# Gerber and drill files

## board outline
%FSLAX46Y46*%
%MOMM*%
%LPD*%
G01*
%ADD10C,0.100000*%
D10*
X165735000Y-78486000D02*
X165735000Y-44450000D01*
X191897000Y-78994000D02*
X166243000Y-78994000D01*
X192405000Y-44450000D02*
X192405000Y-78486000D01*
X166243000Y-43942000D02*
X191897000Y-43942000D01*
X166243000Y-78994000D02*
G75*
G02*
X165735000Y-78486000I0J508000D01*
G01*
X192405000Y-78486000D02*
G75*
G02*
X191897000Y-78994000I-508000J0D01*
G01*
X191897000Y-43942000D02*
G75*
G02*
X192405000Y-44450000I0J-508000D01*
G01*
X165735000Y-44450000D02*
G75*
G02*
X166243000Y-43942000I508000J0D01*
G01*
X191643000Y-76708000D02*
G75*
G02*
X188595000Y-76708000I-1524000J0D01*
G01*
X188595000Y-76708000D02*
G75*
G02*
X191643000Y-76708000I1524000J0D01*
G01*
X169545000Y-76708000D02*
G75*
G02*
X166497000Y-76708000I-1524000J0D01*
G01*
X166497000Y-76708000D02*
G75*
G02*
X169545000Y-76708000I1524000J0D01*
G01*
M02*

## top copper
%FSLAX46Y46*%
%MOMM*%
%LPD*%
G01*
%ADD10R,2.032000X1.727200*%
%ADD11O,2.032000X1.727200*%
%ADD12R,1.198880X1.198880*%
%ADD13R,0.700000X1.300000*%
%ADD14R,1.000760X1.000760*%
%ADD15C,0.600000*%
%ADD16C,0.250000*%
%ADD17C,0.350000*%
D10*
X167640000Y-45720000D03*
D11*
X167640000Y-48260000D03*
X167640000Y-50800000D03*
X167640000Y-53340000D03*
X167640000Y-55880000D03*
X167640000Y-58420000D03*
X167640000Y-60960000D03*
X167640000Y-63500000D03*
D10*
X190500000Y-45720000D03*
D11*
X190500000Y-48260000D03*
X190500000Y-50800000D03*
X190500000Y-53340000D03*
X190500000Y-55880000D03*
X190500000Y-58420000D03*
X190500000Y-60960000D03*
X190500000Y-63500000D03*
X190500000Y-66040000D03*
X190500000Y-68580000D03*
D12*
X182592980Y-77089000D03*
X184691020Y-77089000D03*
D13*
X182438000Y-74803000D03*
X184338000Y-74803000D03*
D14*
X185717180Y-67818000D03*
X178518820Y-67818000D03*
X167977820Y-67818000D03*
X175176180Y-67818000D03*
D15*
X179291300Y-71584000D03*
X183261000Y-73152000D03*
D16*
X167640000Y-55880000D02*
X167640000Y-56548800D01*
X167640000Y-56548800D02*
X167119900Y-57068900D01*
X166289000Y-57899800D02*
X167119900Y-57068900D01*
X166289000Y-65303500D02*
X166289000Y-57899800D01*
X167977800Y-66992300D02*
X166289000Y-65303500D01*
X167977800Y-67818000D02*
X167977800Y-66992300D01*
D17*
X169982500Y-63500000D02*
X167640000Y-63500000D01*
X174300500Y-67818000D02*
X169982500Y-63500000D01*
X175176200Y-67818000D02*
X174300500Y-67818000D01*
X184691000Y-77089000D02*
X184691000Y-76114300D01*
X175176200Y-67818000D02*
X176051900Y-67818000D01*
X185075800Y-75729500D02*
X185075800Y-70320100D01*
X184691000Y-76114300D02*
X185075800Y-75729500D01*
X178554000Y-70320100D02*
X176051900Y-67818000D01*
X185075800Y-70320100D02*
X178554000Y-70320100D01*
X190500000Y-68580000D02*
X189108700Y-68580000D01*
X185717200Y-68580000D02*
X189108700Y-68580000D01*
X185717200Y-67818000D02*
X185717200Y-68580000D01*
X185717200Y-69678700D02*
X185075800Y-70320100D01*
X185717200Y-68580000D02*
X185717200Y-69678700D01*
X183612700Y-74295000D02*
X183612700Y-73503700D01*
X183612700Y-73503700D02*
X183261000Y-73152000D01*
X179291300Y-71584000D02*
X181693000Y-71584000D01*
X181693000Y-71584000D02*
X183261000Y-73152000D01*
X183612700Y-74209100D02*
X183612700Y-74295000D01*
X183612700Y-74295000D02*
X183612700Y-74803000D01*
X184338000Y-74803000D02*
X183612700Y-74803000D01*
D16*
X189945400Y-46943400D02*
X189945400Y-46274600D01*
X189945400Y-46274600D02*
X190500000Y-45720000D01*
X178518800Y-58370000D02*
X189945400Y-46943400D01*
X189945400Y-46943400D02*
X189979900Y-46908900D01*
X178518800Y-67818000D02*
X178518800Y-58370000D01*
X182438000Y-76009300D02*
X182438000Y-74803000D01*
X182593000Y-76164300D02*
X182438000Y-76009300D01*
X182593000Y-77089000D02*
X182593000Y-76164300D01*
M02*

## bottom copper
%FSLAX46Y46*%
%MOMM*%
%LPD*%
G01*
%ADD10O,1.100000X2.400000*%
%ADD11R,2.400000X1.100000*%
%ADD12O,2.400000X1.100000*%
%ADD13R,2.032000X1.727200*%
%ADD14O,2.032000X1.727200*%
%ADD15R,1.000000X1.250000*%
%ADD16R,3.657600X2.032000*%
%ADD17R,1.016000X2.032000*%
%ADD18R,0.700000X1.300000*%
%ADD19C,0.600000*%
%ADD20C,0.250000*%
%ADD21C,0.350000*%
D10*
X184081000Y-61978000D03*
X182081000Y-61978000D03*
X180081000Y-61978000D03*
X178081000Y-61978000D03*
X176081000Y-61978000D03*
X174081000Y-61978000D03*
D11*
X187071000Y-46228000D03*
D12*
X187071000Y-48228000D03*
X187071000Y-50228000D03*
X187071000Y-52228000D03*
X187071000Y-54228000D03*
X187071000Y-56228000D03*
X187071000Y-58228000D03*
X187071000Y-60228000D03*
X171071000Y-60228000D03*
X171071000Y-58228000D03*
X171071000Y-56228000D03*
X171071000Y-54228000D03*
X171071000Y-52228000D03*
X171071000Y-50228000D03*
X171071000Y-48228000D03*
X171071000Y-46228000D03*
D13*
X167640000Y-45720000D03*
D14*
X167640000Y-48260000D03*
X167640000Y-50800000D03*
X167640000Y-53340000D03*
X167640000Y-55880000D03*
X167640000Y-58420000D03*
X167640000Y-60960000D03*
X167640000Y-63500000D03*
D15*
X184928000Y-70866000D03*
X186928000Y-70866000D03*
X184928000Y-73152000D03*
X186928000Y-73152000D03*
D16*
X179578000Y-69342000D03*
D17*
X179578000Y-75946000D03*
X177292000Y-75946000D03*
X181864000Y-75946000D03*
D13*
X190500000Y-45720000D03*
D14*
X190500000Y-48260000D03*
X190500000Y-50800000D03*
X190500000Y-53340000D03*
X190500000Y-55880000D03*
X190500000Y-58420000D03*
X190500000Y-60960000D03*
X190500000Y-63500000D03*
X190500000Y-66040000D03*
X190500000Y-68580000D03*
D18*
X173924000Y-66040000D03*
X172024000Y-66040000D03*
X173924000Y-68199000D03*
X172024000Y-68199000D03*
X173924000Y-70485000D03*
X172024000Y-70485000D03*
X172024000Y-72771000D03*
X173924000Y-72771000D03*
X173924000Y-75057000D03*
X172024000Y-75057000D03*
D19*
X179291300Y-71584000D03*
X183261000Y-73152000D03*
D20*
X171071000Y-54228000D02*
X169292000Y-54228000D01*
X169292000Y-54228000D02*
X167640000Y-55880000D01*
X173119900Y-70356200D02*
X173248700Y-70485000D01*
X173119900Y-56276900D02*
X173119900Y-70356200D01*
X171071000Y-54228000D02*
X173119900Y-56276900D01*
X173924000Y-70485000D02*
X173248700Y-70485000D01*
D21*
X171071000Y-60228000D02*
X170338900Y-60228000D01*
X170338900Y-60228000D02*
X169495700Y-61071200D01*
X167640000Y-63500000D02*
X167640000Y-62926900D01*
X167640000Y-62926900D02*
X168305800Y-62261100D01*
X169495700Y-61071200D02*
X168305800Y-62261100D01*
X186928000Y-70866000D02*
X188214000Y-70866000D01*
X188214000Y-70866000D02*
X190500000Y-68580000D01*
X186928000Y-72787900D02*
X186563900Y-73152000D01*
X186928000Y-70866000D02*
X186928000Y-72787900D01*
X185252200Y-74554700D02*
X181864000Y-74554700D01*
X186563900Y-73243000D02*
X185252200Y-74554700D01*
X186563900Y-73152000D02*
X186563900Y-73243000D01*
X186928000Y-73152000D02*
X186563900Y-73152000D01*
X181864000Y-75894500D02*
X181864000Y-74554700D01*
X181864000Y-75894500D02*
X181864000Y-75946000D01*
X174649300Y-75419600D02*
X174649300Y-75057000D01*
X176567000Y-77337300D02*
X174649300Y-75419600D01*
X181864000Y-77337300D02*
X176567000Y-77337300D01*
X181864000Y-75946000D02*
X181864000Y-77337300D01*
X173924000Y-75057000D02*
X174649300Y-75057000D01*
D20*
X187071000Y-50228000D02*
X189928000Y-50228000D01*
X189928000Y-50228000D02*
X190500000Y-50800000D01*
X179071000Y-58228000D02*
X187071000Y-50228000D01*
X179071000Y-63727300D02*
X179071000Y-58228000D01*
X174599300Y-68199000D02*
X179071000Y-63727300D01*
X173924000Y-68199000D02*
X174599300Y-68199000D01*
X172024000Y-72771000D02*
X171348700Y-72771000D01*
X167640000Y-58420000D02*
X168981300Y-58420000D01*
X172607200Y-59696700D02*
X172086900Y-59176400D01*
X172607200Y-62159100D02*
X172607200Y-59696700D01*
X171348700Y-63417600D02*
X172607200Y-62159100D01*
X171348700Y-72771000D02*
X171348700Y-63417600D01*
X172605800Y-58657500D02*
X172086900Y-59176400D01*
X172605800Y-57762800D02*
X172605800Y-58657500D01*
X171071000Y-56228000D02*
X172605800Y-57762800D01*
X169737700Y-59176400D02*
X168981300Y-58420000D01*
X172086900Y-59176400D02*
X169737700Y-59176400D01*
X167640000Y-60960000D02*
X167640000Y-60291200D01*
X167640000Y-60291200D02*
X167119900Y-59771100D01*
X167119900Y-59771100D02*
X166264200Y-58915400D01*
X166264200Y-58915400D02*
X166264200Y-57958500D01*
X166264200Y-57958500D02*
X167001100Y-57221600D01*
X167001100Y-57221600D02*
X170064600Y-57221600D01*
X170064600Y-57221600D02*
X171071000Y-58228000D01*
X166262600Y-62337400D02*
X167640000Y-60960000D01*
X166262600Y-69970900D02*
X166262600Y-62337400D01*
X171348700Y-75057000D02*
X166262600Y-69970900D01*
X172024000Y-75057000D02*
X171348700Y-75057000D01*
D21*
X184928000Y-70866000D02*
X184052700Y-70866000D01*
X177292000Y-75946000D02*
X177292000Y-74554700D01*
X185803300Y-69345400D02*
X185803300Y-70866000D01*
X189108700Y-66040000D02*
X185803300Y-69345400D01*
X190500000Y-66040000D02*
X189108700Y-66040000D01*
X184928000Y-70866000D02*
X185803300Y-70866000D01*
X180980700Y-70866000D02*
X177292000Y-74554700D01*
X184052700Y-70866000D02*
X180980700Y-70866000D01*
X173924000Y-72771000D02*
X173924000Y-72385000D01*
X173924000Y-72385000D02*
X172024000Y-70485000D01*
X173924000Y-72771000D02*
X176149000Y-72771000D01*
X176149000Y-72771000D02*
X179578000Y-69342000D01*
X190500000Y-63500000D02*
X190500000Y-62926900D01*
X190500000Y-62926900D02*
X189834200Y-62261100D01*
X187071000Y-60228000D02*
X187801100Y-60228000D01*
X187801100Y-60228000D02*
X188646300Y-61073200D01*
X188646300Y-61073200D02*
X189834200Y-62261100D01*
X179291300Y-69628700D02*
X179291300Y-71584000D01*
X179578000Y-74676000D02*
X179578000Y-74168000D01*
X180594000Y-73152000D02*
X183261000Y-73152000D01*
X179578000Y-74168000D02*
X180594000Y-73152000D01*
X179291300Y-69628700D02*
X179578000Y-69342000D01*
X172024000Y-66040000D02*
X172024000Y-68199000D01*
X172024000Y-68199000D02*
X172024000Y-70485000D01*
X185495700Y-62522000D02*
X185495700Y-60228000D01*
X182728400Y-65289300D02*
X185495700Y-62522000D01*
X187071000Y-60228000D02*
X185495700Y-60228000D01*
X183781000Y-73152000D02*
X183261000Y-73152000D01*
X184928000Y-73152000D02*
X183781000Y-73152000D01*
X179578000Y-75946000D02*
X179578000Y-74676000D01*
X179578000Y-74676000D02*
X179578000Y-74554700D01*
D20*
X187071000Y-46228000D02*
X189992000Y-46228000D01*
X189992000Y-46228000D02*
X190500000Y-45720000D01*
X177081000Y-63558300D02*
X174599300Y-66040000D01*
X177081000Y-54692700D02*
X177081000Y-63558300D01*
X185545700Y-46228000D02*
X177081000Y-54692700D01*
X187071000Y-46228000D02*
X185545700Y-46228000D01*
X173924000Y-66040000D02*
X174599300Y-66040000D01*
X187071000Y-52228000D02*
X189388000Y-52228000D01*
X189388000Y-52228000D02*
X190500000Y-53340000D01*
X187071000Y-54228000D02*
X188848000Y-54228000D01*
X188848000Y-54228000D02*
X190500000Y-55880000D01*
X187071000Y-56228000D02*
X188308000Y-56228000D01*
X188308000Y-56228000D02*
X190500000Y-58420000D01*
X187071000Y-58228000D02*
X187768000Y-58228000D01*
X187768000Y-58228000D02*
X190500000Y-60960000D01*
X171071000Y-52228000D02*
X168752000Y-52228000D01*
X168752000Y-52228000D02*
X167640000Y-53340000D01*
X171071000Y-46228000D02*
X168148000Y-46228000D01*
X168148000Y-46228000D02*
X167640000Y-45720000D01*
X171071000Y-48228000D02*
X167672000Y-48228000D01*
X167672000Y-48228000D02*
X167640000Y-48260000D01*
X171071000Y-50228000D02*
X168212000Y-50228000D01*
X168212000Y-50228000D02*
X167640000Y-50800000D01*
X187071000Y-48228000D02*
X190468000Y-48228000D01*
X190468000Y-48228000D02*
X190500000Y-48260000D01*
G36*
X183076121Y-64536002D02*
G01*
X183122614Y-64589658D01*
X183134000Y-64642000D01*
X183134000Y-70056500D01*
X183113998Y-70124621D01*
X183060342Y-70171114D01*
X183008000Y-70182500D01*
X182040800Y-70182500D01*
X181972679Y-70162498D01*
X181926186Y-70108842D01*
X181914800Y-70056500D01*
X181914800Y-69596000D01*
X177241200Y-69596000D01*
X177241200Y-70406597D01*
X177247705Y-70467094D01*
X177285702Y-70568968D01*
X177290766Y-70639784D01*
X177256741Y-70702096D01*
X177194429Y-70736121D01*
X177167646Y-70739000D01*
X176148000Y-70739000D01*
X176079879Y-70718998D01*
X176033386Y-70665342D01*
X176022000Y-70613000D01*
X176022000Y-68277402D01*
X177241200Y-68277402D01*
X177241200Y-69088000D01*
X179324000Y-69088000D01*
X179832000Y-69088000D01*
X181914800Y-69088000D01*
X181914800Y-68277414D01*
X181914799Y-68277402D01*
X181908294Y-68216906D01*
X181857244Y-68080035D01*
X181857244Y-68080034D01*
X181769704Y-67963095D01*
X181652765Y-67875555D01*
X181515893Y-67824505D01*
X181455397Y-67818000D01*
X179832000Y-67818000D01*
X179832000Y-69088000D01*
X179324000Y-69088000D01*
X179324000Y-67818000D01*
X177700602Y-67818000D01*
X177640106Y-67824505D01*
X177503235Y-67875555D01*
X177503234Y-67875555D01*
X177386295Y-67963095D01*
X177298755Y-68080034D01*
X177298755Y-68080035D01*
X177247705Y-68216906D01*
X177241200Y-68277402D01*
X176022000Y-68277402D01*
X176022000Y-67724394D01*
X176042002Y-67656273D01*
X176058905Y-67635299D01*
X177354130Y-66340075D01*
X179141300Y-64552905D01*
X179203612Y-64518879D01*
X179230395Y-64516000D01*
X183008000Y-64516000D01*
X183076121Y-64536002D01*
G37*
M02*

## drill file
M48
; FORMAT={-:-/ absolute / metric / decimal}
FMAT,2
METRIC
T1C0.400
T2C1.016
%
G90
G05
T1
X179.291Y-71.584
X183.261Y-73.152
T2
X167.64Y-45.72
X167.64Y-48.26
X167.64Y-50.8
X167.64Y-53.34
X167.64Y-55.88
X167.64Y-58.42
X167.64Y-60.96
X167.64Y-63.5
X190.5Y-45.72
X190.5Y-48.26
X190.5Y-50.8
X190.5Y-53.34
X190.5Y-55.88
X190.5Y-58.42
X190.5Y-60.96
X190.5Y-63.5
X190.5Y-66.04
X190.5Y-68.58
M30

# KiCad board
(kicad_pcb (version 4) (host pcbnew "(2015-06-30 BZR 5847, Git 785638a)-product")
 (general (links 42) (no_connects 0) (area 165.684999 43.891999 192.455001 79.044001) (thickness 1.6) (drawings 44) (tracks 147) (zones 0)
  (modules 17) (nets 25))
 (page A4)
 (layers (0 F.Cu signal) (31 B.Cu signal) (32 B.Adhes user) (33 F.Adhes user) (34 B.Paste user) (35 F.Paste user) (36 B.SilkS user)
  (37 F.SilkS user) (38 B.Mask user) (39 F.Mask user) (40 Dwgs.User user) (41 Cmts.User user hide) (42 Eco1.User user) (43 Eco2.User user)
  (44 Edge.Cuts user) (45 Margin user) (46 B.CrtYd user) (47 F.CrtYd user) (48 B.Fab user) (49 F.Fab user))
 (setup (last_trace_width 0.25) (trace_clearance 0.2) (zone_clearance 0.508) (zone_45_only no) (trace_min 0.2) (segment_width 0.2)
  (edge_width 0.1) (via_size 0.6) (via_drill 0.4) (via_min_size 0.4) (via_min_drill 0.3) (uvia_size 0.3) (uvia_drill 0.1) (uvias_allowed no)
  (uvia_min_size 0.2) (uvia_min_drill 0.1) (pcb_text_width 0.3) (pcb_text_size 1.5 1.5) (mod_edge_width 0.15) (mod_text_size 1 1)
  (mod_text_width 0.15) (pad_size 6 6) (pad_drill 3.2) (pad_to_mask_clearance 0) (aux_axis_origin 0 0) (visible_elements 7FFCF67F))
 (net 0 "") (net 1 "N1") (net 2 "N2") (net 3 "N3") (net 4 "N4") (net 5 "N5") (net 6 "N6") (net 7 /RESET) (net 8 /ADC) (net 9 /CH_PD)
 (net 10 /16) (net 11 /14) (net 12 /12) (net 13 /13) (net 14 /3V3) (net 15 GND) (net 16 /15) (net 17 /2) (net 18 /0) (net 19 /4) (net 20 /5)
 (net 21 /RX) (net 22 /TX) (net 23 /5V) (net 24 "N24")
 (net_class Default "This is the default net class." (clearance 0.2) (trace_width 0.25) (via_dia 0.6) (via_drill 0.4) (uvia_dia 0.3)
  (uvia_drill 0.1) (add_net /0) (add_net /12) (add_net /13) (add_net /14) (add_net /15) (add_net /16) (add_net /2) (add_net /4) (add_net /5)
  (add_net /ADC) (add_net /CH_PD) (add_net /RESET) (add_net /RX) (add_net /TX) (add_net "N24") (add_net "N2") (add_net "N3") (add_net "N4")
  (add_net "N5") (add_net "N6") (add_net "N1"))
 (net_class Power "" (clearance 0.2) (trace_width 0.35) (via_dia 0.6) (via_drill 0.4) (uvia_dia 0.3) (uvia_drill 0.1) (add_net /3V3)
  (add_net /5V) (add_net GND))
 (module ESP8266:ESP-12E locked (layer B.Cu) (at 187.071 46.228 180)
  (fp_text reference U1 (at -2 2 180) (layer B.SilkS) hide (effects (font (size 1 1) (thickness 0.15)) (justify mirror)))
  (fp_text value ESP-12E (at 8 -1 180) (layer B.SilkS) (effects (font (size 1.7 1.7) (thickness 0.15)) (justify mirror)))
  (pad 9 smd oval (at 2.99 -15.75 90) (size 2.4 1.1) (layers B.Cu B.Paste B.Mask) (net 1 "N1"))
  (pad 10 smd oval (at 4.99 -15.75 90) (size 2.4 1.1) (layers B.Cu B.Paste B.Mask) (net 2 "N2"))
  (pad 11 smd oval (at 6.99 -15.75 90) (size 2.4 1.1) (layers B.Cu B.Paste B.Mask) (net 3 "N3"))
  (pad 12 smd oval (at 8.99 -15.75 90) (size 2.4 1.1) (layers B.Cu B.Paste B.Mask) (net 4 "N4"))
  (pad 13 smd oval (at 10.99 -15.75 90) (size 2.4 1.1) (layers B.Cu B.Paste B.Mask) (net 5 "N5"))
  (pad 14 smd oval (at 12.99 -15.75 90) (size 2.4 1.1) (layers B.Cu B.Paste B.Mask) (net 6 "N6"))
  (pad 1 smd rect (at 0 0 180) (size 2.4 1.1) (layers B.Cu B.Paste B.Mask) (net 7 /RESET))
  (pad 2 smd oval (at 0 -2 180) (size 2.4 1.1) (layers B.Cu B.Paste B.Mask) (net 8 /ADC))
  (pad 3 smd oval (at 0 -4 180) (size 2.4 1.1) (layers B.Cu B.Paste B.Mask) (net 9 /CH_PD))
  (pad 4 smd oval (at 0 -6 180) (size 2.4 1.1) (layers B.Cu B.Paste B.Mask) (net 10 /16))
  (pad 5 smd oval (at 0 -8 180) (size 2.4 1.1) (layers B.Cu B.Paste B.Mask) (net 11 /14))
  (pad 6 smd oval (at 0 -10 180) (size 2.4 1.1) (layers B.Cu B.Paste B.Mask) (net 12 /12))
  (pad 7 smd oval (at 0 -12 180) (size 2.4 1.1) (layers B.Cu B.Paste B.Mask) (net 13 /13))
  (pad 8 smd oval (at 0 -14 180) (size 2.4 1.1) (layers B.Cu B.Paste B.Mask) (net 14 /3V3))
  (pad 15 smd oval (at 16 -14 180) (size 2.4 1.1) (layers B.Cu B.Paste B.Mask) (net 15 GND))
  (pad 16 smd oval (at 16 -12 180) (size 2.4 1.1) (layers B.Cu B.Paste B.Mask) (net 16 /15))
  (pad 17 smd oval (at 16 -10 180) (size 2.4 1.1) (layers B.Cu B.Paste B.Mask) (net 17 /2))
  (pad 18 smd oval (at 16 -8 180) (size 2.4 1.1) (layers B.Cu B.Paste B.Mask) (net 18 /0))
  (pad 19 smd oval (at 16 -6 180) (size 2.4 1.1) (layers B.Cu B.Paste B.Mask) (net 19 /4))
  (pad 20 smd oval (at 16 -4 180) (size 2.4 1.1) (layers B.Cu B.Paste B.Mask) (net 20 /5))
  (pad 21 smd oval (at 16 -2 180) (size 2.4 1.1) (layers B.Cu B.Paste B.Mask) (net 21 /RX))
  (pad 22 smd oval (at 16 0 180) (size 2.4 1.1) (layers B.Cu B.Paste B.Mask) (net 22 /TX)))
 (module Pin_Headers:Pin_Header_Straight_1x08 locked (layer F.Cu) (at 167.64 45.72)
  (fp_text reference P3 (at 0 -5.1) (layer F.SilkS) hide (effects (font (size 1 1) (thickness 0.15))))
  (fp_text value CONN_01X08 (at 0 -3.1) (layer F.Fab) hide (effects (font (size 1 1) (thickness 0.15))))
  (pad 1 thru_hole rect (at 0 0) (size 2.032 1.7272) (drill 1.016) (layers *.Cu *.Mask F.SilkS) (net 22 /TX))
  (pad 2 thru_hole oval (at 0 2.54) (size 2.032 1.7272) (drill 1.016) (layers *.Cu *.Mask F.SilkS) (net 21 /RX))
  (pad 3 thru_hole oval (at 0 5.08) (size 2.032 1.7272) (drill 1.016) (layers *.Cu *.Mask F.SilkS) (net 20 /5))
  (pad 4 thru_hole oval (at 0 7.62) (size 2.032 1.7272) (drill 1.016) (layers *.Cu *.Mask F.SilkS) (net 19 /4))
  (pad 5 thru_hole oval (at 0 10.16) (size 2.032 1.7272) (drill 1.016) (layers *.Cu *.Mask F.SilkS) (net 18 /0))
  (pad 6 thru_hole oval (at 0 12.7) (size 2.032 1.7272) (drill 1.016) (layers *.Cu *.Mask F.SilkS) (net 17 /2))
  (pad 7 thru_hole oval (at 0 15.24) (size 2.032 1.7272) (drill 1.016) (layers *.Cu *.Mask F.SilkS) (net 16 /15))
  (pad 8 thru_hole oval (at 0 17.78) (size 2.032 1.7272) (drill 1.016) (layers *.Cu *.Mask F.SilkS) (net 15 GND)))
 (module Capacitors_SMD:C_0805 (layer B.Cu) (at 185.928 70.866)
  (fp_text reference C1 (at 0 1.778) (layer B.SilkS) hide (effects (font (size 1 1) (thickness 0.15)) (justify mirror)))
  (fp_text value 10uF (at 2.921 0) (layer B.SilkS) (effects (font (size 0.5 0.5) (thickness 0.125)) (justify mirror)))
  (pad 1 smd rect (at -1 0) (size 1 1.25) (layers B.Cu B.Paste B.Mask) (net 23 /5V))
  (pad 2 smd rect (at 1 0) (size 1 1.25) (layers B.Cu B.Paste B.Mask) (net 15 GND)))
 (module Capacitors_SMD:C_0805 (layer B.Cu) (at 185.928 73.152)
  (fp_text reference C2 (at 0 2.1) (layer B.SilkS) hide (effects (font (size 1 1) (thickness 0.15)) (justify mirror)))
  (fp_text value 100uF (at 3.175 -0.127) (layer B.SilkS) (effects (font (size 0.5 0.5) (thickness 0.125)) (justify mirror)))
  (pad 1 smd rect (at -1 0) (size 1 1.25) (layers B.Cu B.Paste B.Mask) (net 14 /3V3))
  (pad 2 smd rect (at 1 0) (size 1 1.25) (layers B.Cu B.Paste B.Mask) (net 15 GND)))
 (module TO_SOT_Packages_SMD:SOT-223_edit (layer B.Cu) (at 179.578 72.644 180)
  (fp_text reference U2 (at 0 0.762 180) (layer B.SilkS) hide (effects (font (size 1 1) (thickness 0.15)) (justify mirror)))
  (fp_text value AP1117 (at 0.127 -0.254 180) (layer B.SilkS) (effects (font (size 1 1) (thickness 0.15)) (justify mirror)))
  (pad 2 smd rect (at 0 3.302 180) (size 3.6576 2.032) (layers B.Cu B.Paste B.Mask) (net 14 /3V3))
  (pad 2 smd rect (at 0 -3.302 180) (size 1.016 2.032) (layers B.Cu B.Paste B.Mask) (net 14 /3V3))
  (pad 3 smd rect (at 2.286 -3.302 180) (size 1.016 2.032) (layers B.Cu B.Paste B.Mask) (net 23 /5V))
  (pad 1 smd rect (at -2.286 -3.302 180) (size 1.016 2.032) (layers B.Cu B.Paste B.Mask) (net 15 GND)))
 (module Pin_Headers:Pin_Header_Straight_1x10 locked (layer F.Cu) (at 190.5 45.72)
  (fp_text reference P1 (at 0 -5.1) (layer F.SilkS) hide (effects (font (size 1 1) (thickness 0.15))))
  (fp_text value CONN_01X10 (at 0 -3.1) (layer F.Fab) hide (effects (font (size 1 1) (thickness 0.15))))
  (pad 1 thru_hole rect (at 0 0) (size 2.032 1.7272) (drill 1.016) (layers *.Cu *.Mask F.SilkS) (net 7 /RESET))
  (pad 2 thru_hole oval (at 0 2.54) (size 2.032 1.7272) (drill 1.016) (layers *.Cu *.Mask F.SilkS) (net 8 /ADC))
  (pad 3 thru_hole oval (at 0 5.08) (size 2.032 1.7272) (drill 1.016) (layers *.Cu *.Mask F.SilkS) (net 9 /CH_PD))
  (pad 4 thru_hole oval (at 0 7.62) (size 2.032 1.7272) (drill 1.016) (layers *.Cu *.Mask F.SilkS) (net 10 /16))
  (pad 5 thru_hole oval (at 0 10.16) (size 2.032 1.7272) (drill 1.016) (layers *.Cu *.Mask F.SilkS) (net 11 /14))
  (pad 6 thru_hole oval (at 0 12.7) (size 2.032 1.7272) (drill 1.016) (layers *.Cu *.Mask F.SilkS) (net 12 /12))
  (pad 7 thru_hole oval (at 0 15.24) (size 2.032 1.7272) (drill 1.016) (layers *.Cu *.Mask F.SilkS) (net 13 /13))
  (pad 8 thru_hole oval (at 0 17.78) (size 2.032 1.7272) (drill 1.016) (layers *.Cu *.Mask F.SilkS) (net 14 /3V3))
  (pad 9 thru_hole oval (at 0 20.32) (size 2.032 1.7272) (drill 1.016) (layers *.Cu *.Mask F.SilkS) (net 23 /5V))
  (pad 10 thru_hole oval (at 0 22.86) (size 2.032 1.7272) (drill 1.016) (layers *.Cu *.Mask F.SilkS) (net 15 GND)))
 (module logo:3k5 (layer F.Cu) (at 180.848 54.864 270)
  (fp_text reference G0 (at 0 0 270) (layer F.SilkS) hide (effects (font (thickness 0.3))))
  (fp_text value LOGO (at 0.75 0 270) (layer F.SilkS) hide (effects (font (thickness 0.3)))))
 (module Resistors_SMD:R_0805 (layer B.Cu) (at 172.974 66.04 180)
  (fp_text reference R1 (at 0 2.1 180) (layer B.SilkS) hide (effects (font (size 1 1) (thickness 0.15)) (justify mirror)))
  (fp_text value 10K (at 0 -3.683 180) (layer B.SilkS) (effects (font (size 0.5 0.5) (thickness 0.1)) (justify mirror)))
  (pad 1 smd rect (at -0.95 0 180) (size 0.7 1.3) (layers B.Cu B.Paste B.Mask) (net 7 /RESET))
  (pad 2 smd rect (at 0.95 0 180) (size 0.7 1.3) (layers B.Cu B.Paste B.Mask) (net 14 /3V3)))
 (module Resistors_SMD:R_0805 (layer B.Cu) (at 172.974 68.199 180)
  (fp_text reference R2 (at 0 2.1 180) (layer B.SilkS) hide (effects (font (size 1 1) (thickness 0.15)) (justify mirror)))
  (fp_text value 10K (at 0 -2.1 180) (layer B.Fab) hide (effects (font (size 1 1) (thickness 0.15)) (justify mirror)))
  (pad 1 smd rect (at -0.95 0 180) (size 0.7 1.3) (layers B.Cu B.Paste B.Mask) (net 9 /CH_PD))
  (pad 2 smd rect (at 0.95 0 180) (size 0.7 1.3) (layers B.Cu B.Paste B.Mask) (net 14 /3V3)))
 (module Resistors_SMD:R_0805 (layer B.Cu) (at 172.974 70.485 180)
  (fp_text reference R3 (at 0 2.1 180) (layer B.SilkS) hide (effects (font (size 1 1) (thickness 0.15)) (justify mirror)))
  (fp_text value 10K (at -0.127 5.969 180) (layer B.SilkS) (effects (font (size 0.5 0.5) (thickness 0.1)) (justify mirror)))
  (pad 1 smd rect (at -0.95 0 180) (size 0.7 1.3) (layers B.Cu B.Paste B.Mask) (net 18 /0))
  (pad 2 smd rect (at 0.95 0 180) (size 0.7 1.3) (layers B.Cu B.Paste B.Mask) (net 14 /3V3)))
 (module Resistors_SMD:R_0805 (layer B.Cu) (at 172.974 72.771)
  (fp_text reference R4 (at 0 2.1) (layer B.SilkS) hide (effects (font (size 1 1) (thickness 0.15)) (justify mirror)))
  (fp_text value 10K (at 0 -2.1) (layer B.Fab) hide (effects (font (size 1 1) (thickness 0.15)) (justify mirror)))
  (pad 1 smd rect (at -0.95 0) (size 0.7 1.3) (layers B.Cu B.Paste B.Mask) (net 17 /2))
  (pad 2 smd rect (at 0.95 0) (size 0.7 1.3) (layers B.Cu B.Paste B.Mask) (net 14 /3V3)))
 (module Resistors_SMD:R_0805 (layer B.Cu) (at 172.974 75.057 180)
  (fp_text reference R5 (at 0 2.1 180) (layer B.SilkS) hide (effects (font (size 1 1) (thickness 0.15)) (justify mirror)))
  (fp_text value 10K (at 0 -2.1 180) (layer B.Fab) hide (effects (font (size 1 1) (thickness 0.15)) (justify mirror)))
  (pad 1 smd rect (at -0.95 0 180) (size 0.7 1.3) (layers B.Cu B.Paste B.Mask) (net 15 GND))
  (pad 2 smd rect (at 0.95 0 180) (size 0.7 1.3) (layers B.Cu B.Paste B.Mask) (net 16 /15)))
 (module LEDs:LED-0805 (layer F.Cu) (at 183.642 77.089 180)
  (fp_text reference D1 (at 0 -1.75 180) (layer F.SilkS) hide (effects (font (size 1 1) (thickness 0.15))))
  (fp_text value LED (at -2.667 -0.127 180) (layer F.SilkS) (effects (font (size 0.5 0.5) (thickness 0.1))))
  (pad 2 smd rect (at 1.04902 0) (size 1.19888 1.19888) (layers F.Cu F.Paste F.Mask) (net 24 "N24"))
  (pad 1 smd rect (at -1.04902 0) (size 1.19888 1.19888) (layers F.Cu F.Paste F.Mask) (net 15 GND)))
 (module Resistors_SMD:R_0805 (layer F.Cu) (at 183.388 74.803)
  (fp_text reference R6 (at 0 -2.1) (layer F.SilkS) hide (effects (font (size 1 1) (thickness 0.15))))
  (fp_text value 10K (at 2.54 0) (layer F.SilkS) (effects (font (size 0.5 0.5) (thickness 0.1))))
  (pad 1 smd rect (at -0.95 0) (size 0.7 1.3) (layers F.Cu F.Paste F.Mask) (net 24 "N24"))
  (pad 2 smd rect (at 0.95 0) (size 0.7 1.3) (layers F.Cu F.Paste F.Mask) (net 14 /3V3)))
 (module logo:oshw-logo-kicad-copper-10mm (layer F.Cu) (at 175.387 75.184)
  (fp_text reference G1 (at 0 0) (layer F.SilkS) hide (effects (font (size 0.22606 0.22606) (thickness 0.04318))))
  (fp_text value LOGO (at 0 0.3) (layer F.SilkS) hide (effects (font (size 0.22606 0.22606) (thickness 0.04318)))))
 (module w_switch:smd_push (layer F.Cu) (at 182.118 67.818 180) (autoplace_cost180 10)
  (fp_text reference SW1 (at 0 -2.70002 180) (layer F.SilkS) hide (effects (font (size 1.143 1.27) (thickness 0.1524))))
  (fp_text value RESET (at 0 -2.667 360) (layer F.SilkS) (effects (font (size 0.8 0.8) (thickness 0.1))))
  (pad 1 smd rect (at -3.59918 0 180) (size 1.00076 1.00076) (layers F.Cu F.Paste F.Mask) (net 15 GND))
  (pad 2 smd rect (at 3.59918 0 180) (size 1.00076 1.00076) (layers F.Cu F.Paste F.Mask) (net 7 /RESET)))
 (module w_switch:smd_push (layer F.Cu) (at 171.577 67.818) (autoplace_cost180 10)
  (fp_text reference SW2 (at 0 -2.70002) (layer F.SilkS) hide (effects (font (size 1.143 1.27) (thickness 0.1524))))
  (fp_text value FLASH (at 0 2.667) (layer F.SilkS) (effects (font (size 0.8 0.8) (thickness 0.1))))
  (pad 1 smd rect (at -3.59918 0) (size 1.00076 1.00076) (layers F.Cu F.Paste F.Mask) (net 18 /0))
  (pad 2 smd rect (at 3.59918 0) (size 1.00076 1.00076) (layers F.Cu F.Paste F.Mask) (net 15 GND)))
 (gr_line (start 165.735 78.486) (end 165.735 44.45) (angle 90) (layer Edge.Cuts) (width 0.1))
 (gr_line (start 191.897 78.994) (end 166.243 78.994) (angle 90) (layer Edge.Cuts) (width 0.1))
 (gr_line (start 192.405 44.45) (end 192.405 78.486) (angle 90) (layer Edge.Cuts) (width 0.1))
 (gr_line (start 166.243 43.942) (end 191.897 43.942) (angle 90) (layer Edge.Cuts) (width 0.1))
 (gr_arc (start 166.243 78.486) (end 166.243 78.994) (angle 90) (layer Edge.Cuts) (width 0.1))
 (gr_arc (start 191.897 78.486) (end 192.405 78.486) (angle 90) (layer Edge.Cuts) (width 0.1))
 (gr_arc (start 191.897 44.45) (end 191.897 43.942) (angle 90) (layer Edge.Cuts) (width 0.1))
 (gr_arc (start 166.243 44.45) (end 165.735 44.45) (angle 90) (layer Edge.Cuts) (width 0.1))
 (gr_circle (center 190.119 76.708) (end 191.643 76.708) (layer Edge.Cuts) (width 0.1))
 (gr_circle (center 168.021 76.708) (end 169.545 76.708) (layer Edge.Cuts) (width 0.1))
 (segment (start 171.071 54.228) (end 169.292 54.228) (width 0.25) (layer B.Cu) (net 18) (status 400000))
 (segment (start 169.292 54.228) (end 167.64 55.88) (width 0.25) (layer B.Cu) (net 18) (status 800000))
 (segment (start 167.64 55.88) (end 167.64 56.5488) (width 0.25) (layer F.Cu) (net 18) (status C00000))
 (segment (start 167.64 56.5488) (end 167.1199 57.0689) (width 0.25) (layer F.Cu) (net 18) (status 400000))
 (segment (start 166.289 57.8998) (end 167.1199 57.0689) (width 0.25) (layer F.Cu) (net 18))
 (segment (start 166.289 65.3035) (end 166.289 57.8998) (width 0.25) (layer F.Cu) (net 18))
 (segment (start 167.9778 66.9923) (end 166.289 65.3035) (width 0.25) (layer F.Cu) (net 18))
 (segment (start 167.9778 67.818) (end 167.9778 66.9923) (width 0.25) (layer F.Cu) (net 18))
 (segment (start 173.1199 70.3562) (end 173.2487 70.485) (width 0.25) (layer B.Cu) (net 18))
 (segment (start 173.1199 56.2769) (end 173.1199 70.3562) (width 0.25) (layer B.Cu) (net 18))
 (segment (start 171.071 54.228) (end 173.1199 56.2769) (width 0.25) (layer B.Cu) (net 18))
 (segment (start 173.924 70.485) (end 173.2487 70.485) (width 0.25) (layer B.Cu) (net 18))
 (segment (start 171.071 60.228) (end 170.3389 60.228) (width 0.35) (layer B.Cu) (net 15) (status C00000))
 (segment (start 170.3389 60.228) (end 169.4957 61.0712) (width 0.35) (layer B.Cu) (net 15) (status 400000))
 (segment (start 167.64 63.5) (end 167.64 62.9269) (width 0.35) (layer B.Cu) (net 15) (status C00000))
 (segment (start 167.64 62.9269) (end 168.3058 62.2611) (width 0.35) (layer B.Cu) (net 15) (status 400000))
 (segment (start 169.4957 61.0712) (end 168.3058 62.2611) (width 0.35) (layer B.Cu) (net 15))
 (segment (start 186.928 70.866) (end 188.214 70.866) (width 0.35) (layer B.Cu) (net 15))
 (segment (start 188.214 70.866) (end 190.5 68.58) (width 0.35) (layer B.Cu) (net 15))
 (segment (start 169.9825 63.5) (end 167.64 63.5) (width 0.35) (layer F.Cu) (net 15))
 (segment (start 174.3005 67.818) (end 169.9825 63.5) (width 0.35) (layer F.Cu) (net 15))
 (segment (start 175.1762 67.818) (end 174.3005 67.818) (width 0.35) (layer F.Cu) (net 15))
 (segment (start 184.691 77.089) (end 184.691 76.1143) (width 0.35) (layer F.Cu) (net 15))
 (segment (start 175.1762 67.818) (end 176.0519 67.818) (width 0.35) (layer F.Cu) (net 15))
 (segment (start 185.0758 75.7295) (end 185.0758 70.3201) (width 0.35) (layer F.Cu) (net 15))
 (segment (start 184.691 76.1143) (end 185.0758 75.7295) (width 0.35) (layer F.Cu) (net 15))
 (segment (start 178.554 70.3201) (end 176.0519 67.818) (width 0.35) (layer F.Cu) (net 15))
 (segment (start 185.0758 70.3201) (end 178.554 70.3201) (width 0.35) (layer F.Cu) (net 15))
 (segment (start 186.928 72.7879) (end 186.5639 73.152) (width 0.35) (layer B.Cu) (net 15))
 (segment (start 186.928 70.866) (end 186.928 72.7879) (width 0.35) (layer B.Cu) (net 15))
 (segment (start 185.2522 74.5547) (end 181.864 74.5547) (width 0.35) (layer B.Cu) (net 15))
 (segment (start 186.5639 73.243) (end 185.2522 74.5547) (width 0.35) (layer B.Cu) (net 15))
 (segment (start 186.5639 73.152) (end 186.5639 73.243) (width 0.35) (layer B.Cu) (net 15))
 (segment (start 186.928 73.152) (end 186.5639 73.152) (width 0.35) (layer B.Cu) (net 15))
 (segment (start 190.5 68.58) (end 189.1087 68.58) (width 0.35) (layer F.Cu) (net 15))
 (segment (start 185.7172 68.58) (end 189.1087 68.58) (width 0.35) (layer F.Cu) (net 15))
 (segment (start 185.7172 67.818) (end 185.7172 68.58) (width 0.35) (layer F.Cu) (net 15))
 (segment (start 185.7172 69.6787) (end 185.0758 70.3201) (width 0.35) (layer F.Cu) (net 15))
 (segment (start 185.7172 68.58) (end 185.7172 69.6787) (width 0.35) (layer F.Cu) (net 15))
 (segment (start 181.864 75.8945) (end 181.864 74.5547) (width 0.35) (layer B.Cu) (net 15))
 (segment (start 181.864 75.8945) (end 181.864 75.946) (width 0.35) (layer B.Cu) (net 15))
 (segment (start 174.6493 75.4196) (end 174.6493 75.057) (width 0.35) (layer B.Cu) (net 15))
 (segment (start 176.567 77.3373) (end 174.6493 75.4196) (width 0.35) (layer B.Cu) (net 15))
 (segment (start 181.864 77.3373) (end 176.567 77.3373) (width 0.35) (layer B.Cu) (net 15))
 (segment (start 181.864 75.946) (end 181.864 77.3373) (width 0.35) (layer B.Cu) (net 15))
 (segment (start 173.924 75.057) (end 174.6493 75.057) (width 0.35) (layer B.Cu) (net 15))
 (segment (start 187.071 50.228) (end 189.928 50.228) (width 0.25) (layer B.Cu) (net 9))
 (segment (start 189.928 50.228) (end 190.5 50.8) (width 0.25) (layer B.Cu) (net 9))
 (segment (start 179.071 58.228) (end 187.071 50.228) (width 0.25) (layer B.Cu) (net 9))
 (segment (start 179.071 63.7273) (end 179.071 58.228) (width 0.25) (layer B.Cu) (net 9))
 (segment (start 174.5993 68.199) (end 179.071 63.7273) (width 0.25) (layer B.Cu) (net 9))
 (segment (start 173.924 68.199) (end 174.5993 68.199) (width 0.25) (layer B.Cu) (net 9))
 (segment (start 172.024 72.771) (end 171.3487 72.771) (width 0.25) (layer B.Cu) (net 17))
 (segment (start 167.64 58.42) (end 168.9813 58.42) (width 0.25) (layer B.Cu) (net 17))
 (segment (start 172.6072 59.6967) (end 172.0869 59.1764) (width 0.25) (layer B.Cu) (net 17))
 (segment (start 172.6072 62.1591) (end 172.6072 59.6967) (width 0.25) (layer B.Cu) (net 17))
 (segment (start 171.3487 63.4176) (end 172.6072 62.1591) (width 0.25) (layer B.Cu) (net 17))
 (segment (start 171.3487 72.771) (end 171.3487 63.4176) (width 0.25) (layer B.Cu) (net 17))
 (segment (start 172.6058 58.6575) (end 172.0869 59.1764) (width 0.25) (layer B.Cu) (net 17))
 (segment (start 172.6058 57.7628) (end 172.6058 58.6575) (width 0.25) (layer B.Cu) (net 17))
 (segment (start 171.071 56.228) (end 172.6058 57.7628) (width 0.25) (layer B.Cu) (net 17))
 (segment (start 169.7377 59.1764) (end 168.9813 58.42) (width 0.25) (layer B.Cu) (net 17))
 (segment (start 172.0869 59.1764) (end 169.7377 59.1764) (width 0.25) (layer B.Cu) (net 17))
 (segment (start 167.64 60.96) (end 167.64 60.2912) (width 0.25) (layer B.Cu) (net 16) (status C00000))
 (segment (start 167.64 60.2912) (end 167.1199 59.7711) (width 0.25) (layer B.Cu) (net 16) (status 400000))
 (segment (start 167.1199 59.7711) (end 166.2642 58.9154) (width 0.25) (layer B.Cu) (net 16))
 (segment (start 166.2642 58.9154) (end 166.2642 57.9585) (width 0.25) (layer B.Cu) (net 16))
 (segment (start 166.2642 57.9585) (end 167.0011 57.2216) (width 0.25) (layer B.Cu) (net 16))
 (segment (start 167.0011 57.2216) (end 170.0646 57.2216) (width 0.25) (layer B.Cu) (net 16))
 (segment (start 170.0646 57.2216) (end 171.071 58.228) (width 0.25) (layer B.Cu) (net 16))
 (segment (start 166.2626 62.3374) (end 167.64 60.96) (width 0.25) (layer B.Cu) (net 16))
 (segment (start 166.2626 69.9709) (end 166.2626 62.3374) (width 0.25) (layer B.Cu) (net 16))
 (segment (start 171.3487 75.057) (end 166.2626 69.9709) (width 0.25) (layer B.Cu) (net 16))
 (segment (start 172.024 75.057) (end 171.3487 75.057) (width 0.25) (layer B.Cu) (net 16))
 (segment (start 184.928 70.866) (end 184.0527 70.866) (width 0.35) (layer B.Cu) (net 23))
 (segment (start 177.292 75.946) (end 177.292 74.5547) (width 0.35) (layer B.Cu) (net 23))
 (segment (start 185.8033 69.3454) (end 185.8033 70.866) (width 0.35) (layer B.Cu) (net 23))
 (segment (start 189.1087 66.04) (end 185.8033 69.3454) (width 0.35) (layer B.Cu) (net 23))
 (segment (start 190.5 66.04) (end 189.1087 66.04) (width 0.35) (layer B.Cu) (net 23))
 (segment (start 184.928 70.866) (end 185.8033 70.866) (width 0.35) (layer B.Cu) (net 23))
 (segment (start 180.9807 70.866) (end 177.292 74.5547) (width 0.35) (layer B.Cu) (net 23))
 (segment (start 184.0527 70.866) (end 180.9807 70.866) (width 0.35) (layer B.Cu) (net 23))
 (segment (start 173.924 72.771) (end 173.924 72.385) (width 0.35) (layer B.Cu) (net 14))
 (segment (start 173.924 72.385) (end 172.024 70.485) (width 0.35) (layer B.Cu) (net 14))
 (segment (start 173.924 72.771) (end 176.149 72.771) (width 0.35) (layer B.Cu) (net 14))
 (segment (start 176.149 72.771) (end 179.578 69.342) (width 0.35) (layer B.Cu) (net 14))
 (segment (start 190.5 63.5) (end 190.5 62.9269) (width 0.35) (layer B.Cu) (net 14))
 (segment (start 190.5 62.9269) (end 189.8342 62.2611) (width 0.35) (layer B.Cu) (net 14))
 (segment (start 187.071 60.228) (end 187.8011 60.228) (width 0.35) (layer B.Cu) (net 14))
 (segment (start 187.8011 60.228) (end 188.6463 61.0732) (width 0.35) (layer B.Cu) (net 14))
 (segment (start 188.6463 61.0732) (end 189.8342 62.2611) (width 0.35) (layer B.Cu) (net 14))
 (segment (start 183.6127 74.295) (end 183.6127 73.5037) (width 0.35) (layer F.Cu) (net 14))
 (segment (start 183.6127 73.5037) (end 183.261 73.152) (width 0.35) (layer F.Cu) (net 14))
 (segment (start 179.2913 71.584) (end 181.693 71.584) (width 0.35) (layer F.Cu) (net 14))
 (segment (start 181.693 71.584) (end 183.261 73.152) (width 0.35) (layer F.Cu) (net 14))
 (segment (start 179.2913 69.6287) (end 179.2913 71.584) (width 0.35) (layer B.Cu) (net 14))
 (via (at 179.2913 71.584) (size 0.6) (layers F.Cu B.Cu) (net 14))
 (segment (start 179.578 74.676) (end 179.578 74.168) (width 0.35) (layer B.Cu) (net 14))
 (segment (start 180.594 73.152) (end 183.261 73.152) (width 0.35) (layer B.Cu) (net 14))
 (segment (start 179.578 74.168) (end 180.594 73.152) (width 0.35) (layer B.Cu) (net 14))
 (via (at 183.261 73.152) (size 0.6) (layers F.Cu B.Cu) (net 14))
 (segment (start 179.2913 69.6287) (end 179.578 69.342) (width 0.35) (layer B.Cu) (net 14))
 (segment (start 172.024 66.04) (end 172.024 68.199) (width 0.35) (layer B.Cu) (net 14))
 (segment (start 172.024 68.199) (end 172.024 70.485) (width 0.35) (layer B.Cu) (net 14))
 (segment (start 185.4957 62.522) (end 185.4957 60.228) (width 0.35) (layer B.Cu) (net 14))
 (segment (start 182.7284 65.2893) (end 185.4957 62.522) (width 0.35) (layer B.Cu) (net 14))
 (segment (start 187.071 60.228) (end 185.4957 60.228) (width 0.35) (layer B.Cu) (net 14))
 (segment (start 183.781 73.152) (end 183.261 73.152) (width 0.35) (layer B.Cu) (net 14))
 (segment (start 184.928 73.152) (end 183.781 73.152) (width 0.35) (layer B.Cu) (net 14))
 (segment (start 183.6127 74.2091) (end 183.6127 74.295) (width 0.35) (layer F.Cu) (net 14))
 (segment (start 183.6127 74.295) (end 183.6127 74.803) (width 0.35) (layer F.Cu) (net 14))
 (segment (start 184.338 74.803) (end 183.6127 74.803) (width 0.35) (layer F.Cu) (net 14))
 (segment (start 179.578 75.946) (end 179.578 74.676) (width 0.35) (layer B.Cu) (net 14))
 (segment (start 179.578 74.676) (end 179.578 74.5547) (width 0.35) (layer B.Cu) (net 14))
 (segment (start 189.9454 46.9434) (end 189.9454 46.2746) (width 0.25) (layer F.Cu) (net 7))
 (segment (start 189.9454 46.2746) (end 190.5 45.72) (width 0.25) (layer F.Cu) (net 7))
 (segment (start 187.071 46.228) (end 189.992 46.228) (width 0.25) (layer B.Cu) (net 7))
 (segment (start 189.992 46.228) (end 190.5 45.72) (width 0.25) (layer B.Cu) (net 7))
 (segment (start 178.5188 58.37) (end 189.9454 46.9434) (width 0.25) (layer F.Cu) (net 7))
 (segment (start 189.9454 46.9434) (end 189.9799 46.9089) (width 0.25) (layer F.Cu) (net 7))
 (segment (start 178.5188 67.818) (end 178.5188 58.37) (width 0.25) (layer F.Cu) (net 7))
 (segment (start 177.081 63.5583) (end 174.5993 66.04) (width 0.25) (layer B.Cu) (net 7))
 (segment (start 177.081 54.6927) (end 177.081 63.5583) (width 0.25) (layer B.Cu) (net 7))
 (segment (start 185.5457 46.228) (end 177.081 54.6927) (width 0.25) (layer B.Cu) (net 7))
 (segment (start 187.071 46.228) (end 185.5457 46.228) (width 0.25) (layer B.Cu) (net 7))
 (segment (start 173.924 66.04) (end 174.5993 66.04) (width 0.25) (layer B.Cu) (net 7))
 (segment (start 187.071 52.228) (end 189.388 52.228) (width 0.25) (layer B.Cu) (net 10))
 (segment (start 189.388 52.228) (end 190.5 53.34) (width 0.25) (layer B.Cu) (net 10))
 (segment (start 187.071 54.228) (end 188.848 54.228) (width 0.25) (layer B.Cu) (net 11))
 (segment (start 188.848 54.228) (end 190.5 55.88) (width 0.25) (layer B.Cu) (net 11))
 (segment (start 187.071 56.228) (end 188.308 56.228) (width 0.25) (layer B.Cu) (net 12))
 (segment (start 188.308 56.228) (end 190.5 58.42) (width 0.25) (layer B.Cu) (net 12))
 (segment (start 187.071 58.228) (end 187.768 58.228) (width 0.25) (layer B.Cu) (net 13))
 (segment (start 187.768 58.228) (end 190.5 60.96) (width 0.25) (layer B.Cu) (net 13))
 (segment (start 171.071 52.228) (end 168.752 52.228) (width 0.25) (layer B.Cu) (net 19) (status 400000))
 (segment (start 168.752 52.228) (end 167.64 53.34) (width 0.25) (layer B.Cu) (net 19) (status 800000))
 (segment (start 171.071 46.228) (end 168.148 46.228) (width 0.25) (layer B.Cu) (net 22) (status C00000))
 (segment (start 168.148 46.228) (end 167.64 45.72) (width 0.25) (layer B.Cu) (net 22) (status C00000))
 (segment (start 171.071 48.228) (end 167.672 48.228) (width 0.25) (layer B.Cu) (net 21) (status C00000))
 (segment (start 167.672 48.228) (end 167.64 48.26) (width 0.25) (layer B.Cu) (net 21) (status C00000))
 (segment (start 171.071 50.228) (end 168.212 50.228) (width 0.25) (layer B.Cu) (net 20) (status C00000))
 (segment (start 168.212 50.228) (end 167.64 50.8) (width 0.25) (layer B.Cu) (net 20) (status C00000))
 (segment (start 187.071 48.228) (end 190.468 48.228) (width 0.25) (layer B.Cu) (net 8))
 (segment (start 190.468 48.228) (end 190.5 48.26) (width 0.25) (layer B.Cu) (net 8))
 (segment (start 182.438 76.0093) (end 182.438 74.803) (width 0.25) (layer F.Cu) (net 24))
 (segment (start 182.593 76.1643) (end 182.438 76.0093) (width 0.25) (layer F.Cu) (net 24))
 (segment (start 182.593 77.089) (end 182.593 76.1643) (width 0.25) (layer F.Cu) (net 24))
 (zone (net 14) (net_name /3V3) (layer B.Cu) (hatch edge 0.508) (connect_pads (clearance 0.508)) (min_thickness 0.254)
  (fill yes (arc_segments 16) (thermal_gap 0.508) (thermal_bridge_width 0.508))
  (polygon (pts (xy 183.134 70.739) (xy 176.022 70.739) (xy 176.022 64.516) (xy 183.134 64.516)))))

